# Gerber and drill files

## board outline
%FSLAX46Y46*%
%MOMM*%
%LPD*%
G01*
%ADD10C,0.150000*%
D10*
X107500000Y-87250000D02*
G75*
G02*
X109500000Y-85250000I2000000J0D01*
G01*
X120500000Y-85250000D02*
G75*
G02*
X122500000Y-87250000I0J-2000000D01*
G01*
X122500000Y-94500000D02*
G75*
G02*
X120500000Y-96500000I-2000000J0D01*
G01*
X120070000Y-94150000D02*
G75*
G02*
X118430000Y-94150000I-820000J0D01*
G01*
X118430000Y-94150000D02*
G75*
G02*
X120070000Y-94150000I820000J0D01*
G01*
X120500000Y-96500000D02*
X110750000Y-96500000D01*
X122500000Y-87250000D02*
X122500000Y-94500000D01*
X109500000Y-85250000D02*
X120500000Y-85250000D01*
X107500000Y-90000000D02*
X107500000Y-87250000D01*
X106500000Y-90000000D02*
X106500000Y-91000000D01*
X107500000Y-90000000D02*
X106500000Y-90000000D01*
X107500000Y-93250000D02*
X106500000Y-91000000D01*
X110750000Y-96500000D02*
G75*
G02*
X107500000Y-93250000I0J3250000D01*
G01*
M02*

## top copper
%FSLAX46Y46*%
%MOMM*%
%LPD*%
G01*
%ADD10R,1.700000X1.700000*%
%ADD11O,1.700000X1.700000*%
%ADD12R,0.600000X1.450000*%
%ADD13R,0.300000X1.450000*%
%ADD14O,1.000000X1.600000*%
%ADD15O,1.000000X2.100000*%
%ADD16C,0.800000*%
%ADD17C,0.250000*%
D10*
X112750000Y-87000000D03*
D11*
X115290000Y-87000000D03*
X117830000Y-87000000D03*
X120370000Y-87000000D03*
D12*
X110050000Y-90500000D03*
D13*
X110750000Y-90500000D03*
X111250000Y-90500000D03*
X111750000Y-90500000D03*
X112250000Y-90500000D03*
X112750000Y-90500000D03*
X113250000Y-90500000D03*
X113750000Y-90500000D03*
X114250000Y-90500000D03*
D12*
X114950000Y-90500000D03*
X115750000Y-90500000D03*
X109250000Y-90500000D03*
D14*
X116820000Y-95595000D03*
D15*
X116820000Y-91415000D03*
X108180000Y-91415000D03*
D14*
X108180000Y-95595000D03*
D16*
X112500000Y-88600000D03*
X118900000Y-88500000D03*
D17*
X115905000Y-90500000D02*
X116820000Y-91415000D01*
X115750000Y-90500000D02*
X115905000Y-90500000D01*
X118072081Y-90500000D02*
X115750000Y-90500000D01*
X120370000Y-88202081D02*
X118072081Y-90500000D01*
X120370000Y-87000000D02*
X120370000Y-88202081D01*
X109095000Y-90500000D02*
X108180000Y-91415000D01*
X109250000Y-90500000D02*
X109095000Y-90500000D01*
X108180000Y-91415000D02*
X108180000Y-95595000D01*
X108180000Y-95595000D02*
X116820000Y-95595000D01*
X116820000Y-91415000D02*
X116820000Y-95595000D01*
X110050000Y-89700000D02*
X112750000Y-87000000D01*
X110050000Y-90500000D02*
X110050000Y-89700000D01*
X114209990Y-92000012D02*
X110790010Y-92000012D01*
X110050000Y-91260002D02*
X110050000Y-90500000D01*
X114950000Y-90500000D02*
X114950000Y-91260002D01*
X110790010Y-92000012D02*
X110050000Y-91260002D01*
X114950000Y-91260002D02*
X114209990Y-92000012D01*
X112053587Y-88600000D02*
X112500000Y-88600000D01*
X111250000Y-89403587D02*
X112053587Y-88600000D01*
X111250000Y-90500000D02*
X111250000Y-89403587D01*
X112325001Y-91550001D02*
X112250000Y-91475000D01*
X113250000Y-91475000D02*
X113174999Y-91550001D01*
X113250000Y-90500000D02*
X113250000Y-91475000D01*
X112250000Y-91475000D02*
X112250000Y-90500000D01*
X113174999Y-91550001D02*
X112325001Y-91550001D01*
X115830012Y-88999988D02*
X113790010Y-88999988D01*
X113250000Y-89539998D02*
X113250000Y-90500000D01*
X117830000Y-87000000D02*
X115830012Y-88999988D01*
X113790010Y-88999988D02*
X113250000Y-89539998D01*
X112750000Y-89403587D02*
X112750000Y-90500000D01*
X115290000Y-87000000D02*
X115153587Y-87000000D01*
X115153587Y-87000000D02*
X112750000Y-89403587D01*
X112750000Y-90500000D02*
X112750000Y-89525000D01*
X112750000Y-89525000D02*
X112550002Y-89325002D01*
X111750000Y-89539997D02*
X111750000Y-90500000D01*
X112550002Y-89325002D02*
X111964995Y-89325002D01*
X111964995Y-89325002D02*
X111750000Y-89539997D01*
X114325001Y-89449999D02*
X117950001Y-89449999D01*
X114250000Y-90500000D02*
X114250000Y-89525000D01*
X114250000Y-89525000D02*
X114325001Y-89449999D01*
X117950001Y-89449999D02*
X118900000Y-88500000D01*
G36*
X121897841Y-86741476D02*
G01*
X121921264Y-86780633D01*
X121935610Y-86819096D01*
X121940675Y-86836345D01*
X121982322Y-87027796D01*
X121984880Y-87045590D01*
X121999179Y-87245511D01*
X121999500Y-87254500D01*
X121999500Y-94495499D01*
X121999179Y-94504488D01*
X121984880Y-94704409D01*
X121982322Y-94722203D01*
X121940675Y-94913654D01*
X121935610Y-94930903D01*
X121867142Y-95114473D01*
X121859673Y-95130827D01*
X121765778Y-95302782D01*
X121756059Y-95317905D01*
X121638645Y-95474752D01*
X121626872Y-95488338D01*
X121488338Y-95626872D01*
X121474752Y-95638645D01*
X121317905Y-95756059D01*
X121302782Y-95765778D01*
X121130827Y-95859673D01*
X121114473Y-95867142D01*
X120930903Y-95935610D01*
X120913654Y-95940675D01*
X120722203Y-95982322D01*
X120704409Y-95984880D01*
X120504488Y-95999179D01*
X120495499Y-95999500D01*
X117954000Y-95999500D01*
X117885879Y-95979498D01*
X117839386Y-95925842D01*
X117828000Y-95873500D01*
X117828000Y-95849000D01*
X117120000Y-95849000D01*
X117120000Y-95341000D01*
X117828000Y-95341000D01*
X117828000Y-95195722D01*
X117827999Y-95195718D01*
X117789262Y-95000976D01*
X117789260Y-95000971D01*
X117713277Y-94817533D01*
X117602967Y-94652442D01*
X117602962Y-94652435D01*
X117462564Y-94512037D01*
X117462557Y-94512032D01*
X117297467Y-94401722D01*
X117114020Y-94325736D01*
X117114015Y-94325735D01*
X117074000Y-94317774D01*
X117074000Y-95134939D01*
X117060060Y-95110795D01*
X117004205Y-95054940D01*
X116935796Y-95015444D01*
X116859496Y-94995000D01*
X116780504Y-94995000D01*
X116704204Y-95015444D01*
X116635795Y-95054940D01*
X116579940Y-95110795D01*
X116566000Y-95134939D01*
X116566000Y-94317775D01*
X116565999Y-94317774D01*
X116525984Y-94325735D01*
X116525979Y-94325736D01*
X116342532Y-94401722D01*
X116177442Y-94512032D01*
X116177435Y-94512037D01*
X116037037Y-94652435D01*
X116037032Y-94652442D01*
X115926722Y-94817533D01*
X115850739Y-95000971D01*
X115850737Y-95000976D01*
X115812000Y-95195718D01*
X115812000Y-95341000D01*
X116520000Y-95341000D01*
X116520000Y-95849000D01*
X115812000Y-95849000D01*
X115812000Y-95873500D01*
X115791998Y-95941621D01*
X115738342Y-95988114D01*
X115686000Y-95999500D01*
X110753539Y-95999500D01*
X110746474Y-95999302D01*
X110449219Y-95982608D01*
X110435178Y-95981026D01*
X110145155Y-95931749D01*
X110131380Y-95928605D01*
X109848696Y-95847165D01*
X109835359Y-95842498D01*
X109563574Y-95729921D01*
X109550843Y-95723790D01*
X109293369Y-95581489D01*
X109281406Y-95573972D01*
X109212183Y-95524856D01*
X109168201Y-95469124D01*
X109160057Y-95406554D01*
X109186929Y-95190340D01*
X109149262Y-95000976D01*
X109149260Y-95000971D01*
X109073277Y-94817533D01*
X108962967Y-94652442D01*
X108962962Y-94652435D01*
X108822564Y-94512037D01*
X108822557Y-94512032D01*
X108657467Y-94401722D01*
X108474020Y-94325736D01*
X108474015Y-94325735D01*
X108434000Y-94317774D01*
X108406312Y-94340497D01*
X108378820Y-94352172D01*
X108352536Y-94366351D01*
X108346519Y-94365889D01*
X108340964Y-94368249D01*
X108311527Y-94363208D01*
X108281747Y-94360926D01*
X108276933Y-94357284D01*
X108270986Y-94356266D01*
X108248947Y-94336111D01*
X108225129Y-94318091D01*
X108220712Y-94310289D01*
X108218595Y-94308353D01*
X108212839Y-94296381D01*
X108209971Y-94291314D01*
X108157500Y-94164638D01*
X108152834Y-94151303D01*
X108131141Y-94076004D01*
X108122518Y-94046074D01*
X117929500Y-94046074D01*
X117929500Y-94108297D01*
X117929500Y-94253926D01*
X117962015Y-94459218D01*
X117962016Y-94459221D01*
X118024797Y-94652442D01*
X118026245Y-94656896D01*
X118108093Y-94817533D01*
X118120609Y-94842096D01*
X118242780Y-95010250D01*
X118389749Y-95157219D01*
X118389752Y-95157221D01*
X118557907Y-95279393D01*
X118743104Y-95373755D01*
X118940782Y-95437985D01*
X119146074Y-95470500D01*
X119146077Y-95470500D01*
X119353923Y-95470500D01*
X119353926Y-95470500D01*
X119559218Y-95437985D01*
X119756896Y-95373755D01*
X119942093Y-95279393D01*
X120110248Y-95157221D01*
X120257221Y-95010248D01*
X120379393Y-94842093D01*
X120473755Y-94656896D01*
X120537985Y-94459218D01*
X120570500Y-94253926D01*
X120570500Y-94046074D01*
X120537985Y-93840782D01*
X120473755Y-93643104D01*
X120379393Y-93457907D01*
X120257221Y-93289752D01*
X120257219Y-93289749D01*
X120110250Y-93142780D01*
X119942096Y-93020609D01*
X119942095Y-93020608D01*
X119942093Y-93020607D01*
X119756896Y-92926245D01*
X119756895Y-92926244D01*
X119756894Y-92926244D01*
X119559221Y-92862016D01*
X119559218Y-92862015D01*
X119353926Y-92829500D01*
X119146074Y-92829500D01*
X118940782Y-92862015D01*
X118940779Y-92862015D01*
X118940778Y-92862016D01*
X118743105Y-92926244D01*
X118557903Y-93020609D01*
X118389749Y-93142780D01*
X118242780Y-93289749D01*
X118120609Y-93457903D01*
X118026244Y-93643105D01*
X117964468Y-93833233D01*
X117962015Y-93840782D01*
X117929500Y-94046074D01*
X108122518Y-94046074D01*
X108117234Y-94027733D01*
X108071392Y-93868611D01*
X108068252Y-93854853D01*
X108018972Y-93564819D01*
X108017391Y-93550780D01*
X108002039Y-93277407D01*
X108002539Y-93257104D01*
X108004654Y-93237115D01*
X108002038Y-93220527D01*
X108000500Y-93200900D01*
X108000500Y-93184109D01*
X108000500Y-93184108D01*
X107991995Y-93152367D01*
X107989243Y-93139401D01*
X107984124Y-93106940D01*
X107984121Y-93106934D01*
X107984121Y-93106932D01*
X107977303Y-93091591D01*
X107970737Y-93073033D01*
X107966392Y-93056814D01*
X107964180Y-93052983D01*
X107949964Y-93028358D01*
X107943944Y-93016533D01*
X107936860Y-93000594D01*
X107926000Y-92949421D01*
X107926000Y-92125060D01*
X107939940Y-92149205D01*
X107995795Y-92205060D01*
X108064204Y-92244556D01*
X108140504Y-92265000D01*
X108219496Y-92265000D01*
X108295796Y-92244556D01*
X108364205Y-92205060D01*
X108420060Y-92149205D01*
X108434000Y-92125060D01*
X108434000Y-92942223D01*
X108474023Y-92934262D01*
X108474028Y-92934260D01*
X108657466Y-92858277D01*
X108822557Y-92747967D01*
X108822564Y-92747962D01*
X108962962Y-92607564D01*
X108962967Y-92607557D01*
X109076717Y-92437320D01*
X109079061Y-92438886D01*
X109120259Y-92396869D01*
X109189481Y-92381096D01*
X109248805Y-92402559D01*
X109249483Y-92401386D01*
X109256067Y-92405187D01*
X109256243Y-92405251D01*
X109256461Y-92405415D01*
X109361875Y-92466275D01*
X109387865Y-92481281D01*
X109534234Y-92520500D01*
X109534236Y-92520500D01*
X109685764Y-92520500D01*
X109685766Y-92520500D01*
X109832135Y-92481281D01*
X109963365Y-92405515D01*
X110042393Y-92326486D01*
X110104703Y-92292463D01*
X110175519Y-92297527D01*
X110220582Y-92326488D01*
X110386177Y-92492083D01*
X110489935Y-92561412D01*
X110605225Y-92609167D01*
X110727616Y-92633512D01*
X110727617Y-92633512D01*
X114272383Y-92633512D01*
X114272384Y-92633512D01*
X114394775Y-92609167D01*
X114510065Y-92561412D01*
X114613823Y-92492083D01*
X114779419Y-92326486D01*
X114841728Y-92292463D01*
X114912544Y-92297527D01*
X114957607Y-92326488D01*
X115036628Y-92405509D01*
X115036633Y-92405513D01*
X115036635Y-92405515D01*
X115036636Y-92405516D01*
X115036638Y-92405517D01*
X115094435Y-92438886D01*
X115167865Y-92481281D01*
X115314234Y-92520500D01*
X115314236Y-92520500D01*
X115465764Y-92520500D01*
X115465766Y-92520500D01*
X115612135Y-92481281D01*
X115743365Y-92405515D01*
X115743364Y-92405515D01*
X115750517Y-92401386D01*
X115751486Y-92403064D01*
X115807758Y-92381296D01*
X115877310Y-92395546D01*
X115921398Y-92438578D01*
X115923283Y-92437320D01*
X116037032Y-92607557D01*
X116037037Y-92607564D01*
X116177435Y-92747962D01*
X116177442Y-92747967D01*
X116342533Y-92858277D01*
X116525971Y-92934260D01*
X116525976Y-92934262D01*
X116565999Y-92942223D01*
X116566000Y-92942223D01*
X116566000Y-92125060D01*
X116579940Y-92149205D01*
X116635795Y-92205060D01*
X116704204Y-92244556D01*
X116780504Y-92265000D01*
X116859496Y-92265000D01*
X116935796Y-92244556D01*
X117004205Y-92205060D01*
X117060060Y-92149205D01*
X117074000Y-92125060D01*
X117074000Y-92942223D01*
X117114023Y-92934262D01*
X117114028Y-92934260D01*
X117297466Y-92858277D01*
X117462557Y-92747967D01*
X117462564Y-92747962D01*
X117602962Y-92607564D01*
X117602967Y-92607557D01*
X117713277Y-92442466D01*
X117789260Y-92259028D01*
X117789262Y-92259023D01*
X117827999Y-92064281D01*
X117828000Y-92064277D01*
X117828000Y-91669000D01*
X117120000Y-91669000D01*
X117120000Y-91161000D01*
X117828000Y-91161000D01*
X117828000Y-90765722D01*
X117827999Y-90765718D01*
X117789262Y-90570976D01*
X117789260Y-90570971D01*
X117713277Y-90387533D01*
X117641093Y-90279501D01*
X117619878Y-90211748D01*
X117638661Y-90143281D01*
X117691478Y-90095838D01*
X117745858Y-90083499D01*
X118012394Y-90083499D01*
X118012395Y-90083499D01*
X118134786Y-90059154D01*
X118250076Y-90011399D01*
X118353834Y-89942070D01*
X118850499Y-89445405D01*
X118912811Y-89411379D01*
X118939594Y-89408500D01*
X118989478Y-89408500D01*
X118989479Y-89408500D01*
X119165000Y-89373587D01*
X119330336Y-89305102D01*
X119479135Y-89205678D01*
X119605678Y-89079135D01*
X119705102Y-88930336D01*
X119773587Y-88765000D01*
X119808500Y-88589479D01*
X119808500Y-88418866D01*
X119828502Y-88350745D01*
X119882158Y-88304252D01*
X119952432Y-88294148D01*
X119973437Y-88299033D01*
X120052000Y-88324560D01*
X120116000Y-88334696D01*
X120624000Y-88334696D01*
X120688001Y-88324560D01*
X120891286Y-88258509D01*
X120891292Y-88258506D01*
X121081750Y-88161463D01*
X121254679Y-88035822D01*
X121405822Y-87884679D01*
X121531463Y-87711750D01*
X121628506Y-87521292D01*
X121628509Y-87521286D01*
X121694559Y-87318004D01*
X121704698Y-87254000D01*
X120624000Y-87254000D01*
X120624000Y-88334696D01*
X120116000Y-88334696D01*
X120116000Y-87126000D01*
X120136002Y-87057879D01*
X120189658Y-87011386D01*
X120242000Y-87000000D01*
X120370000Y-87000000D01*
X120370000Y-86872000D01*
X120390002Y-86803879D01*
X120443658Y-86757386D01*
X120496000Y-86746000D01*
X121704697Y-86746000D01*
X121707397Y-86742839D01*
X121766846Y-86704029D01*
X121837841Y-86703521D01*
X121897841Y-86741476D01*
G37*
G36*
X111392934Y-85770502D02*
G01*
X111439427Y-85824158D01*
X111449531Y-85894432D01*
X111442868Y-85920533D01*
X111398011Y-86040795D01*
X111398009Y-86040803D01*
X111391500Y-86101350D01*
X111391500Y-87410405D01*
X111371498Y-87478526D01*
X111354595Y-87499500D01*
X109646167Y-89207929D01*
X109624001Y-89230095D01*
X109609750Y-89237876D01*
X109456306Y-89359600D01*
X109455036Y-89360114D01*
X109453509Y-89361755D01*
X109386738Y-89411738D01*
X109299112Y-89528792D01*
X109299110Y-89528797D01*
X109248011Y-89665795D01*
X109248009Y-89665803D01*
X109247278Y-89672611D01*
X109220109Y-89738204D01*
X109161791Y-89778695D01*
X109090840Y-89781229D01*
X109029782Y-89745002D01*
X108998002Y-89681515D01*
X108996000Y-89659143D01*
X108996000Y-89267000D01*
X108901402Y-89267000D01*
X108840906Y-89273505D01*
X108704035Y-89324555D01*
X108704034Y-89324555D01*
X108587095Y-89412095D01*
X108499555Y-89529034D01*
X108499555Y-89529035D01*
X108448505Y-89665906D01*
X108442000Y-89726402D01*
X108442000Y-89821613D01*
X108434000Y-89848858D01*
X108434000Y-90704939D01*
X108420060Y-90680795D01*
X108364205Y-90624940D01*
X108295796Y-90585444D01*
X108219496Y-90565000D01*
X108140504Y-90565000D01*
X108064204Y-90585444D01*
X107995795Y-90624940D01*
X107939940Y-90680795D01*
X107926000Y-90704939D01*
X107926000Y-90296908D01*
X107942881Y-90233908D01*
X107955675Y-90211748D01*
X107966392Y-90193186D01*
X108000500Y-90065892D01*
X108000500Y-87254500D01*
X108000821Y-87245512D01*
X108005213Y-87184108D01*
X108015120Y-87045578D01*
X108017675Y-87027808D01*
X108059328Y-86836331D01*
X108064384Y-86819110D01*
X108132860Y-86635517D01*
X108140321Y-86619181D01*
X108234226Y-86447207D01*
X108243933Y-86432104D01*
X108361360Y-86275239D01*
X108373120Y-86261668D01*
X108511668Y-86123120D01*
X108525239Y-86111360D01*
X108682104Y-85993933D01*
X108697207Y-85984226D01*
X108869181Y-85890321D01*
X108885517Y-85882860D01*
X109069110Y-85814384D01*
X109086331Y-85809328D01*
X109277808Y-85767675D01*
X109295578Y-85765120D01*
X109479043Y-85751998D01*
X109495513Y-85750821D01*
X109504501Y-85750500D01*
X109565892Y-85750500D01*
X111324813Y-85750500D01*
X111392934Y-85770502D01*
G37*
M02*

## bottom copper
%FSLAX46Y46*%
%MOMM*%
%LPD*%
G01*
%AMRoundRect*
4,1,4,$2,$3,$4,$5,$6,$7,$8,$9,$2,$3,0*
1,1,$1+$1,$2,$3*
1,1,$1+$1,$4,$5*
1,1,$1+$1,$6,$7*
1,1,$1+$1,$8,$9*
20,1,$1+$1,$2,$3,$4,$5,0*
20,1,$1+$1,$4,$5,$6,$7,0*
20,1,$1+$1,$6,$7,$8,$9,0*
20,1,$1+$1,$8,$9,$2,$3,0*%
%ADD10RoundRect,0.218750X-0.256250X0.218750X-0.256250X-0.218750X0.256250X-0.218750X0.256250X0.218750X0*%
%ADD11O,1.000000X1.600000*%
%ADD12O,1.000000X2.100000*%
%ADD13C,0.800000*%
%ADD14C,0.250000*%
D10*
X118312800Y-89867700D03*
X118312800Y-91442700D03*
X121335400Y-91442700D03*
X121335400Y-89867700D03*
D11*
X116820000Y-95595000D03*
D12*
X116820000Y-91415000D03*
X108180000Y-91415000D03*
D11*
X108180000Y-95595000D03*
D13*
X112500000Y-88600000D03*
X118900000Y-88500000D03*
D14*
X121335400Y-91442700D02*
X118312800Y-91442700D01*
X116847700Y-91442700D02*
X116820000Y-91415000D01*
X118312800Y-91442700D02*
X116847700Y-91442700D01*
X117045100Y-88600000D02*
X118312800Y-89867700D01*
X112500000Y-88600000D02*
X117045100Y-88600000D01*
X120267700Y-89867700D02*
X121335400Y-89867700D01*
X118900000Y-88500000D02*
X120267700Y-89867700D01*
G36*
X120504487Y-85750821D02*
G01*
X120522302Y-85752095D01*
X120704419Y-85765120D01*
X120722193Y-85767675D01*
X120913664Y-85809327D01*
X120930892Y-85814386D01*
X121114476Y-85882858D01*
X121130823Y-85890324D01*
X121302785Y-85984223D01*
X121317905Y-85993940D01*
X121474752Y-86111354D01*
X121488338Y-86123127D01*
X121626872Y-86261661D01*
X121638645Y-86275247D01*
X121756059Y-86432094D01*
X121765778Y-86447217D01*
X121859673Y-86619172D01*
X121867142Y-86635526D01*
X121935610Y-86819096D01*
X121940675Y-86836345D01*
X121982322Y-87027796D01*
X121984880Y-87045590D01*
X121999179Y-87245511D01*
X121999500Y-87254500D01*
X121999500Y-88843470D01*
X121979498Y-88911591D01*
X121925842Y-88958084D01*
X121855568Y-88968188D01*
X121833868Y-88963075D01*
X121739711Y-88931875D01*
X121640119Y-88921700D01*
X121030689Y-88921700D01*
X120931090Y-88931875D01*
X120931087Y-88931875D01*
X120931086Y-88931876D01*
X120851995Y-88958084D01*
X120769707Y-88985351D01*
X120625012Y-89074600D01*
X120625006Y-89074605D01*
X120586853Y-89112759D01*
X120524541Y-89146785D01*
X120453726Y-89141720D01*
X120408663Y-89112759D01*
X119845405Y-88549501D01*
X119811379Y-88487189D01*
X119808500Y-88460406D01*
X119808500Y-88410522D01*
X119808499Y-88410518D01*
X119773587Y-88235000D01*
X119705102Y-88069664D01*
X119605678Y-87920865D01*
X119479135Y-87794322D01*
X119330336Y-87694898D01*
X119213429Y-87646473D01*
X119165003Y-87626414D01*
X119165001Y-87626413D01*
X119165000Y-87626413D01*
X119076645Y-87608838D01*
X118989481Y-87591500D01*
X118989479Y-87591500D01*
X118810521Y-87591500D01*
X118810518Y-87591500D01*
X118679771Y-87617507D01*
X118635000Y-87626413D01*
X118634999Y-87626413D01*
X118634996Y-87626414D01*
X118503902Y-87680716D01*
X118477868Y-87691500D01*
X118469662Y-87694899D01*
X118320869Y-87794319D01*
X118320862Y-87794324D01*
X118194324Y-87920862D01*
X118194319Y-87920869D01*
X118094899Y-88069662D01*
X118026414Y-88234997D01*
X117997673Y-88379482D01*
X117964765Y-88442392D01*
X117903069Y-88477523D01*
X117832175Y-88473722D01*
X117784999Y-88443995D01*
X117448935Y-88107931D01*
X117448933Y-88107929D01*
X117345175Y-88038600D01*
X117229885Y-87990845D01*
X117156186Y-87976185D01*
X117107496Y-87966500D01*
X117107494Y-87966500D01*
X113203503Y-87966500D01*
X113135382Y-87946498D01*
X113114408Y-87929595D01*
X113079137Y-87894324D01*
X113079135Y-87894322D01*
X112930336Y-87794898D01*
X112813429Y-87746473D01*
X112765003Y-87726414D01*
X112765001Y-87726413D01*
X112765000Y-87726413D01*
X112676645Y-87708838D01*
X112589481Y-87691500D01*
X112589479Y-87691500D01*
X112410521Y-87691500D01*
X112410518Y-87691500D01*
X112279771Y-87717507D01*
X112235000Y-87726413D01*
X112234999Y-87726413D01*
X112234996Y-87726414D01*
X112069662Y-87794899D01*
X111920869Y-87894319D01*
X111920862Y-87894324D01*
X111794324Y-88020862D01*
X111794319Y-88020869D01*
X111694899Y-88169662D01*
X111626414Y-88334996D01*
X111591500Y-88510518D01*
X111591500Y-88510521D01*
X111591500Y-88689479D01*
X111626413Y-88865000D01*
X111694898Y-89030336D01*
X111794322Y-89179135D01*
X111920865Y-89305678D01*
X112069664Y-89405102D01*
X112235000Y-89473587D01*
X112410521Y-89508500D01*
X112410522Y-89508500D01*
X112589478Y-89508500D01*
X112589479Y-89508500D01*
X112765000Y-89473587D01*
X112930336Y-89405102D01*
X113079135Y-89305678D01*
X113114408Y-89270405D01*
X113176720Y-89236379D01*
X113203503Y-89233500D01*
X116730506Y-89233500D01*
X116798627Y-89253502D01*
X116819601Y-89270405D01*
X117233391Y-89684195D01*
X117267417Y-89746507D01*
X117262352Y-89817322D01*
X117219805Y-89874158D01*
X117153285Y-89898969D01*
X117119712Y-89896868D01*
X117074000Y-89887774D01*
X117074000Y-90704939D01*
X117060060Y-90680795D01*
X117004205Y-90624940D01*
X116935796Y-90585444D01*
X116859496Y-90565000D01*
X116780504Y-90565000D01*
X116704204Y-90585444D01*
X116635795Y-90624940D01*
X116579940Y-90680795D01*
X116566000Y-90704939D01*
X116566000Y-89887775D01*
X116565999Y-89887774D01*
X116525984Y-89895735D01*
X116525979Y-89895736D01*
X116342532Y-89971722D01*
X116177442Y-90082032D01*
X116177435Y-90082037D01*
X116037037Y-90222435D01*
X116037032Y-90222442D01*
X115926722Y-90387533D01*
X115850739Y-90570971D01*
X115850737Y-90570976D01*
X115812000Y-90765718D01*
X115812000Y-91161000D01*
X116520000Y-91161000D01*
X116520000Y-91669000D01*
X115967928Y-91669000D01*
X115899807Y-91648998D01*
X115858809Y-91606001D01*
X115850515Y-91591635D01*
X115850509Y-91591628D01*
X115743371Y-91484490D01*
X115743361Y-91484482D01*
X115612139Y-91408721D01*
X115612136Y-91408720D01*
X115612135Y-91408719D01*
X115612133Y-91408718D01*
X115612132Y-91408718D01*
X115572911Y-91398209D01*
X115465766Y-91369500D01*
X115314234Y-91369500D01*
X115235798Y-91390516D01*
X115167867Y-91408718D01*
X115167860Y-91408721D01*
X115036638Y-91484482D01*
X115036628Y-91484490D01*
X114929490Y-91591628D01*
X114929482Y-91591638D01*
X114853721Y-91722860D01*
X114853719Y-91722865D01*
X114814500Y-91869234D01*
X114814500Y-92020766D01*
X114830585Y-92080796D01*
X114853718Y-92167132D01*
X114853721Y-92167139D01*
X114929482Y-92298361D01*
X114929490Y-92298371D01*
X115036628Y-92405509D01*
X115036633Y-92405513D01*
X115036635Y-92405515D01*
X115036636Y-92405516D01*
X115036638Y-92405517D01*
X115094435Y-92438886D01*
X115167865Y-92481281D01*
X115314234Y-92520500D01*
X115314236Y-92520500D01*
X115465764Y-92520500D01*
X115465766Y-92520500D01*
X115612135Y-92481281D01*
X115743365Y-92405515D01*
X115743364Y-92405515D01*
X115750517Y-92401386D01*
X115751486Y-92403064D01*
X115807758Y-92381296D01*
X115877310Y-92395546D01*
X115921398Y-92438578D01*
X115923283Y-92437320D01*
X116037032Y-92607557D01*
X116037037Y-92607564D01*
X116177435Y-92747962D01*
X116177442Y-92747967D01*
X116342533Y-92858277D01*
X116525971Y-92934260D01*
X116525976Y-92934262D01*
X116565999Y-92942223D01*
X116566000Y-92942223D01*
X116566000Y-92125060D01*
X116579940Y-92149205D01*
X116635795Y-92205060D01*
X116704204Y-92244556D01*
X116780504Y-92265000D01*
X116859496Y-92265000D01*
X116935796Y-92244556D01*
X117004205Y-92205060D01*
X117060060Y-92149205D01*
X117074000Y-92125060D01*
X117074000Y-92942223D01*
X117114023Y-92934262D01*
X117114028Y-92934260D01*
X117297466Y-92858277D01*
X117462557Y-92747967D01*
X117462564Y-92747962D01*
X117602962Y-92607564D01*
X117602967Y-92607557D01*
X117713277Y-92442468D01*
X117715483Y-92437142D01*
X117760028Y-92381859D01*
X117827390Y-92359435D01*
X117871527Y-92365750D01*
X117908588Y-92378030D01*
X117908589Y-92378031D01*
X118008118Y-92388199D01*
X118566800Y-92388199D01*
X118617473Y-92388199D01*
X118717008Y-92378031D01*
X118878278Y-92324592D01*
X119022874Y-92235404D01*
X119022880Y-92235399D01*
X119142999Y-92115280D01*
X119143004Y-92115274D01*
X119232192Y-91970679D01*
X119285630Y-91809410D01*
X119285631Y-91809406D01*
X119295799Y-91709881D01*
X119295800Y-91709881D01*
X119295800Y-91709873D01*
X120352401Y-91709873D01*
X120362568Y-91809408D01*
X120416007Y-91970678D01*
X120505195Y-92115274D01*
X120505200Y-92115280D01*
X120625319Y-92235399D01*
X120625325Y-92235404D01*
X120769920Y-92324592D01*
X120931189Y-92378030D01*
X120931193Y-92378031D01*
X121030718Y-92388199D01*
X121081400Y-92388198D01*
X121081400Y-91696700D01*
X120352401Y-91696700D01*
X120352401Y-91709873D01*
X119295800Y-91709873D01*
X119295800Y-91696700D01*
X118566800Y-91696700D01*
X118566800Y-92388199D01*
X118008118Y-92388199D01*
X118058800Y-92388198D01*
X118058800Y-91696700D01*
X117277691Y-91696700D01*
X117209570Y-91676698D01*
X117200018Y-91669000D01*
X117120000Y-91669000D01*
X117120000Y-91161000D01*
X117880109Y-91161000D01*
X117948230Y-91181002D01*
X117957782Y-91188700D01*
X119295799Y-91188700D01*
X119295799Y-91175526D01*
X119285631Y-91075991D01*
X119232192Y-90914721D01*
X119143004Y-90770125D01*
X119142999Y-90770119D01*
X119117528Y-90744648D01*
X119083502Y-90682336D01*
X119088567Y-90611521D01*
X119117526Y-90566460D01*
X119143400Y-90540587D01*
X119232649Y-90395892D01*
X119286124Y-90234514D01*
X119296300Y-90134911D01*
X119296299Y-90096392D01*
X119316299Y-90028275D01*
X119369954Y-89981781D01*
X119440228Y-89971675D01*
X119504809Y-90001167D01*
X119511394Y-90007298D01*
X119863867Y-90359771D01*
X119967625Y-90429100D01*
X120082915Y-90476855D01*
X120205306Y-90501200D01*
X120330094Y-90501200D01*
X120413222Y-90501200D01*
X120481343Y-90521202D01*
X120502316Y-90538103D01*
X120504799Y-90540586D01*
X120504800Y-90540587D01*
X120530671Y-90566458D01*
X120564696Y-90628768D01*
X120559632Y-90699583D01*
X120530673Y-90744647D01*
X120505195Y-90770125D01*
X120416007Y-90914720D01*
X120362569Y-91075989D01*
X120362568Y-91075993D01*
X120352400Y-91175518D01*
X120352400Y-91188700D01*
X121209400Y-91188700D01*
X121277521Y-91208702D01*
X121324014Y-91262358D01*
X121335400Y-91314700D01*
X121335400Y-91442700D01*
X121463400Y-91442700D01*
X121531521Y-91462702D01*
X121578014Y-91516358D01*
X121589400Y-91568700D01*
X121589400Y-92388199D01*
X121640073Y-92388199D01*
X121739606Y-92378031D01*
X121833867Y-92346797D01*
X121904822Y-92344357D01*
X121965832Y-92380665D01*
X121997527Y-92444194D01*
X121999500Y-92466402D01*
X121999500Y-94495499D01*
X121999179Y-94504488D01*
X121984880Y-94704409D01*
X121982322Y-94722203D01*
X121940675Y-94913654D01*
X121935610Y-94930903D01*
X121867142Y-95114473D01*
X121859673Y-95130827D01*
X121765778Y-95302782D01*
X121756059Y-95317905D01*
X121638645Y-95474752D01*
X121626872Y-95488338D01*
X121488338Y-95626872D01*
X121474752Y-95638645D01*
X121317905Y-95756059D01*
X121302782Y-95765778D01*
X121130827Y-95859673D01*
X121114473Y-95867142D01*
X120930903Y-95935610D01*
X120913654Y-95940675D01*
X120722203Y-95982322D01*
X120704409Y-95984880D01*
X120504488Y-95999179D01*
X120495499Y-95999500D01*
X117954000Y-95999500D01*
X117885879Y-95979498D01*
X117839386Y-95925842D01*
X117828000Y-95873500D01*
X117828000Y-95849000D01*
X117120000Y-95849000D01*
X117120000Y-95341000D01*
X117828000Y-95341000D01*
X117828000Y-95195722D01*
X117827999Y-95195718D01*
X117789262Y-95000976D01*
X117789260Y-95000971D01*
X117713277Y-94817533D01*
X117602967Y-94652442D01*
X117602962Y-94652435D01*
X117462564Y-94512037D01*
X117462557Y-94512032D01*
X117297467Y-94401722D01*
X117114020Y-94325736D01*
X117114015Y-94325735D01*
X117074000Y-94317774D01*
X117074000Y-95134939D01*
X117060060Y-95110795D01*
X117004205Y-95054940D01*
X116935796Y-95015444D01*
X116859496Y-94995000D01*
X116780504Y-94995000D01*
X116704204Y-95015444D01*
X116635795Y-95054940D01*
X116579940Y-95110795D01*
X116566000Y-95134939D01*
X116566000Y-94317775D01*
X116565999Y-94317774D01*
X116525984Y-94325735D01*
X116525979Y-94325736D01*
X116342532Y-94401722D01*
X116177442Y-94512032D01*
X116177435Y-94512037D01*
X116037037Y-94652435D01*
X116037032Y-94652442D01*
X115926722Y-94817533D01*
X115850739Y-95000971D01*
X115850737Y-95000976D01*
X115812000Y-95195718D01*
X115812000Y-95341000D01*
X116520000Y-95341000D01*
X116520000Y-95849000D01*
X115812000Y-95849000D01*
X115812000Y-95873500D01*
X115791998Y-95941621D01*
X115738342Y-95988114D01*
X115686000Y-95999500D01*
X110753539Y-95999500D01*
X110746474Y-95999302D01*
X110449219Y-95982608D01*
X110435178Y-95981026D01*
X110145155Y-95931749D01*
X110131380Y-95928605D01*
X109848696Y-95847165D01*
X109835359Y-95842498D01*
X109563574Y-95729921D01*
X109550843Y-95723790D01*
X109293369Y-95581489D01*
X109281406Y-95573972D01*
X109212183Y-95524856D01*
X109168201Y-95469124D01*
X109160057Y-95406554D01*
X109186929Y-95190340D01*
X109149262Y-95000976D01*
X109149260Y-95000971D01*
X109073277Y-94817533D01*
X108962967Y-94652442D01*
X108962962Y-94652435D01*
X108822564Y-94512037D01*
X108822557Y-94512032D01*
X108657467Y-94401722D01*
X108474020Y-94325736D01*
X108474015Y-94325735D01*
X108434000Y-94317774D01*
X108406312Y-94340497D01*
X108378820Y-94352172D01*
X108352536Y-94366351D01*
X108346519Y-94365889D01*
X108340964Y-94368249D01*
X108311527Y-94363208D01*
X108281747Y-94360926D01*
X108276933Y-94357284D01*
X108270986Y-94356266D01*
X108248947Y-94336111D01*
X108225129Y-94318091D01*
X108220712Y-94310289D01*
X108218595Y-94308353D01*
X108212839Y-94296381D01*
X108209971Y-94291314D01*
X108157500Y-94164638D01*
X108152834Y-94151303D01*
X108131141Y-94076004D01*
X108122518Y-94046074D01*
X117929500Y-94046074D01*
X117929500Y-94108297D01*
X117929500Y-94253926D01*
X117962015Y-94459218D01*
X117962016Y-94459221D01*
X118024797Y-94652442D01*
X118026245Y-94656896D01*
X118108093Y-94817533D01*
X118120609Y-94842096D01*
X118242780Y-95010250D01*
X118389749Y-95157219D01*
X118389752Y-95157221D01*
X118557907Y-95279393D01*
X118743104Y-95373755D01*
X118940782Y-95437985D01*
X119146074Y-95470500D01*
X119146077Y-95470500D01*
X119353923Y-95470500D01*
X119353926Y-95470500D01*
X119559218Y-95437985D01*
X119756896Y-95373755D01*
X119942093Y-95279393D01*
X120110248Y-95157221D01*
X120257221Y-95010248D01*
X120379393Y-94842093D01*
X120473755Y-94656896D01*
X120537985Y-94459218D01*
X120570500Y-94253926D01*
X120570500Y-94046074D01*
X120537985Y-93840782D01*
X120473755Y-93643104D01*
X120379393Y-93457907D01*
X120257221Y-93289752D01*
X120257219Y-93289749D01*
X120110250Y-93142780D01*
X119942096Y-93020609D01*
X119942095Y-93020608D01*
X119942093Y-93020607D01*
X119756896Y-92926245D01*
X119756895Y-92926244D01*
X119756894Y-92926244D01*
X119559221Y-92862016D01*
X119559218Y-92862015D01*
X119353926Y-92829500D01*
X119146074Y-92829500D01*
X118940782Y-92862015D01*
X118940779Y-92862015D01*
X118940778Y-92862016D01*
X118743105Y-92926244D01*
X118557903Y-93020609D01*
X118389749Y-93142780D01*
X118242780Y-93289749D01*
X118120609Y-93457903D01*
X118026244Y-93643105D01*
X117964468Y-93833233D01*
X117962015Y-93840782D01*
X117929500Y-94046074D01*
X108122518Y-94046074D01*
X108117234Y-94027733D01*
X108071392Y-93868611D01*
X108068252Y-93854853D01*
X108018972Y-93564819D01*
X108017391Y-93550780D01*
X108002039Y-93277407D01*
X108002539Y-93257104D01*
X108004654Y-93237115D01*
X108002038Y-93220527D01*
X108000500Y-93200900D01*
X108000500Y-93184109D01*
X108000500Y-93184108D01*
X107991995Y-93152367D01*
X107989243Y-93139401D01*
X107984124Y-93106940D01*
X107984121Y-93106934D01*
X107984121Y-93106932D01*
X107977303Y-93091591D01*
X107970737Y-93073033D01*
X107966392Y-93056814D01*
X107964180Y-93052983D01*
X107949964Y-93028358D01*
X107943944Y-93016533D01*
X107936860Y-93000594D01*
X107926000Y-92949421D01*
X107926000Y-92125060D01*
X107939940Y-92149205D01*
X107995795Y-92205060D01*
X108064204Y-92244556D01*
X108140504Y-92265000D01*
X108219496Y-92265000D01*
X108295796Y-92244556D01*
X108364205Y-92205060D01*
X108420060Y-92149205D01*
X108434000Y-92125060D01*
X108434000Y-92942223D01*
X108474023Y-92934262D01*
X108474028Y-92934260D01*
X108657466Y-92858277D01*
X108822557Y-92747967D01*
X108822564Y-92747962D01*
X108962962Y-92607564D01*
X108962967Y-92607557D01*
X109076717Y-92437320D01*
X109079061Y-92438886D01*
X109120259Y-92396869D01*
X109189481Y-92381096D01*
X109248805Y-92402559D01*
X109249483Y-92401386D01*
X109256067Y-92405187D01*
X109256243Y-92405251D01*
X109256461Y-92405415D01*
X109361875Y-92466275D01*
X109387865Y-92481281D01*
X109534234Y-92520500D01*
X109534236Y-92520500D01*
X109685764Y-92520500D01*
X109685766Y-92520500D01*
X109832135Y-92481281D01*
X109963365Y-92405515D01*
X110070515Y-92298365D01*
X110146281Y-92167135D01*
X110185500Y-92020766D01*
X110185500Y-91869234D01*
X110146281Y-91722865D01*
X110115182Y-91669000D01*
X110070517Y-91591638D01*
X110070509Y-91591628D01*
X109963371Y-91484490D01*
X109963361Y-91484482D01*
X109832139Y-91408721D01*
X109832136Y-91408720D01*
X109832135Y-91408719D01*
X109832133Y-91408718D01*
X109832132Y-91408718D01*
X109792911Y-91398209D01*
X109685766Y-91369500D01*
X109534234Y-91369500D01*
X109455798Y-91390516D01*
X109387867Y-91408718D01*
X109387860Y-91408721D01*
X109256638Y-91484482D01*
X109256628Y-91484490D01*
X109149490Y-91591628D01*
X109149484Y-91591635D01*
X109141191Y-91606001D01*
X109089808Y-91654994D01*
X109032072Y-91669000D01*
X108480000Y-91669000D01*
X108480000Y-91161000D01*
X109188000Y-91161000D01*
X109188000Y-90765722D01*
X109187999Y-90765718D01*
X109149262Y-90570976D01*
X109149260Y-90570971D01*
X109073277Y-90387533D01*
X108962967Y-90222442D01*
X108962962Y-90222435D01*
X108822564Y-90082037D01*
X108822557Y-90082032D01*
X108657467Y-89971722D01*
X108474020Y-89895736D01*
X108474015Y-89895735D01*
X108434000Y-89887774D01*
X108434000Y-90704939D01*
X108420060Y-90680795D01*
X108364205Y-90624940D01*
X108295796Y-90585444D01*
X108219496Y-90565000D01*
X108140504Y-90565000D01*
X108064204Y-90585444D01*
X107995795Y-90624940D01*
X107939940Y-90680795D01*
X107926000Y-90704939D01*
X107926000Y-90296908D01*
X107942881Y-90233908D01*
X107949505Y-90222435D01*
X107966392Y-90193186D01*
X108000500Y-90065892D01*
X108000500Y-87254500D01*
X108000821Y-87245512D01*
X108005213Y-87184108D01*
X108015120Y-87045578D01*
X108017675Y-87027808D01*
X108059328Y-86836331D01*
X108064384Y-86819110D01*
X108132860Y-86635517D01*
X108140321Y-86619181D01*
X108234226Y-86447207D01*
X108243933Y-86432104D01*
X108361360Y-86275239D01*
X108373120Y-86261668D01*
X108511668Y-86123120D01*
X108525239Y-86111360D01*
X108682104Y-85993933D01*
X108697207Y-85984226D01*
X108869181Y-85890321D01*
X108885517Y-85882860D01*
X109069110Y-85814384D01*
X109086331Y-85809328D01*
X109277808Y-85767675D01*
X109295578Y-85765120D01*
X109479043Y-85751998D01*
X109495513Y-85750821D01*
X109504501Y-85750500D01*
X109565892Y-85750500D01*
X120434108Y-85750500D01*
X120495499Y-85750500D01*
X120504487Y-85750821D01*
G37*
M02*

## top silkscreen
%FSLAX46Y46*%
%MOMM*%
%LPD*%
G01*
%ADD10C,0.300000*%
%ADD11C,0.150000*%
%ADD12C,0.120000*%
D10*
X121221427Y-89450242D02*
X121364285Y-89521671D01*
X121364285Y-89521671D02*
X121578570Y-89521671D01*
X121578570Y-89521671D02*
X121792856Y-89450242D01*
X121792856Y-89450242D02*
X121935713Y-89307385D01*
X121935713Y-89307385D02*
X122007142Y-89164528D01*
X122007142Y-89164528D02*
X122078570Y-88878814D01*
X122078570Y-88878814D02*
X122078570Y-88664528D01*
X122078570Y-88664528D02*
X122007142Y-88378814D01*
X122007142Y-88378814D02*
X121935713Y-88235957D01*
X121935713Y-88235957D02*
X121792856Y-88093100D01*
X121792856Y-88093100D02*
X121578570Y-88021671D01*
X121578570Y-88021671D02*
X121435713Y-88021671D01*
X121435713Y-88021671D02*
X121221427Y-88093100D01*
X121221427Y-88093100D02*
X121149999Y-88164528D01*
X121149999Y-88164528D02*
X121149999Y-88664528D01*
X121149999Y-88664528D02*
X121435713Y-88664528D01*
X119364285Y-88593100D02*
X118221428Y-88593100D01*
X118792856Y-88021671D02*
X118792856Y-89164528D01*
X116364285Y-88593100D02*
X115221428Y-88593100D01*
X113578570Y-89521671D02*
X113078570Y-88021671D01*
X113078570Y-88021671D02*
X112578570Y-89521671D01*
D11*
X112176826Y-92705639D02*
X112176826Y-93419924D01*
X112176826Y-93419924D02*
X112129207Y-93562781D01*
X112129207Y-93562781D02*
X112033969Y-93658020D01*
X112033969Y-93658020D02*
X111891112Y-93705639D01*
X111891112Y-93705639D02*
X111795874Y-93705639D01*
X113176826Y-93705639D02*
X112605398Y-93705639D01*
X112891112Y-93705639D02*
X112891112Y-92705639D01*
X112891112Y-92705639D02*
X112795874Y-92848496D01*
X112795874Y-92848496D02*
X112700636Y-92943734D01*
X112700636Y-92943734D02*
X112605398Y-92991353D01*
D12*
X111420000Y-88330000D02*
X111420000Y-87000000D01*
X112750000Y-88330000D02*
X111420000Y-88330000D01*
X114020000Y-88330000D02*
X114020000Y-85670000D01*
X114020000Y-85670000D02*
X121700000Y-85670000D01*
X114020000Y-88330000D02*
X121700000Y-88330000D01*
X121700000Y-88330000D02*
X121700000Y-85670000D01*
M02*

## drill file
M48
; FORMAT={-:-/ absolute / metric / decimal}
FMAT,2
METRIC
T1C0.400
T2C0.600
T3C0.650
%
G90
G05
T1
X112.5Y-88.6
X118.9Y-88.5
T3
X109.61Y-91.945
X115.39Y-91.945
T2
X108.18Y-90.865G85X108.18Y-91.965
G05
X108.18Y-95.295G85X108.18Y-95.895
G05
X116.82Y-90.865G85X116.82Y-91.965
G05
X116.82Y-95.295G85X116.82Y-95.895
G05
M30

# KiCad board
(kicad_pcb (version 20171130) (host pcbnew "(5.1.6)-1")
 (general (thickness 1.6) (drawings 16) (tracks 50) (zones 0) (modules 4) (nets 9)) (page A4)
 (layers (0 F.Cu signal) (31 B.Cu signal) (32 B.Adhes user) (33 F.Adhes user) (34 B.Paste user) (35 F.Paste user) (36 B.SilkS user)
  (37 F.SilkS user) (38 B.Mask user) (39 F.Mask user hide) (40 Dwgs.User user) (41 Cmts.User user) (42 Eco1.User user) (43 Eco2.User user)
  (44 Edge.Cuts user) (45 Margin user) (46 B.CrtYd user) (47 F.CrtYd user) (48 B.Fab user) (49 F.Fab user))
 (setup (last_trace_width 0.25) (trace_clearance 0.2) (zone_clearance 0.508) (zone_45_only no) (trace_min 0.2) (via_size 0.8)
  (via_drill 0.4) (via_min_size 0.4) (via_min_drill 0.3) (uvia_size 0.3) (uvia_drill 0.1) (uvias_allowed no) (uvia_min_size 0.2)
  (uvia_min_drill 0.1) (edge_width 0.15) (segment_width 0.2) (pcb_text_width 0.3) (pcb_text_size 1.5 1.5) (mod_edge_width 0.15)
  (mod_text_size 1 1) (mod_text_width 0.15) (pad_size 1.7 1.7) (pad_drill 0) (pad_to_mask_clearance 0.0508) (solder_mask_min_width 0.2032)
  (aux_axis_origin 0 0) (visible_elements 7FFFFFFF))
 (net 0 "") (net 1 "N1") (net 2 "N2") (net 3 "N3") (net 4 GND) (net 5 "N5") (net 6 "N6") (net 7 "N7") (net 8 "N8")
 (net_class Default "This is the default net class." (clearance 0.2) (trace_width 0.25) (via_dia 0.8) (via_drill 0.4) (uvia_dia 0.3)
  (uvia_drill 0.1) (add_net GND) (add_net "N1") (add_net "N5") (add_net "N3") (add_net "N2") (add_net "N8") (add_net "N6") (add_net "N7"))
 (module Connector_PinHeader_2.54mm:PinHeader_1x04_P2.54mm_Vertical (layer F.Cu) (at 112.75 87 90)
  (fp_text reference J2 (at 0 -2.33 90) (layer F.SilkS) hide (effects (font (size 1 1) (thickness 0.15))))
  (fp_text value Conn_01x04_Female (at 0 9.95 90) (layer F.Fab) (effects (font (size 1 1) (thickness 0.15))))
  (fp_line (start -1.33 -1.33) (end 0 -1.33) (layer F.SilkS) (width 0.12))
  (fp_line (start -1.33 0) (end -1.33 -1.33) (layer F.SilkS) (width 0.12))
  (fp_line (start -1.33 1.27) (end 1.33 1.27) (layer F.SilkS) (width 0.12))
  (fp_line (start 1.33 1.27) (end 1.33 8.95) (layer F.SilkS) (width 0.12))
  (fp_line (start -1.33 1.27) (end -1.33 8.95) (layer F.SilkS) (width 0.12))
  (fp_line (start -1.33 8.95) (end 1.33 8.95) (layer F.SilkS) (width 0.12))
  (pad 1 smd rect (at 0 0 90) (size 1.7 1.7) (layers F.Cu F.Paste F.Mask) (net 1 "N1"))
  (pad 2 smd oval (at 0 2.54 90) (size 1.7 1.7) (layers F.Cu F.Paste F.Mask) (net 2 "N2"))
  (pad 3 smd oval (at 0 5.08 90) (size 1.7 1.7) (layers F.Cu F.Paste F.Mask) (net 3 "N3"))
  (pad 4 smd oval (at 0 7.62 90) (size 1.7 1.7) (layers F.Cu F.Paste F.Mask) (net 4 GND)))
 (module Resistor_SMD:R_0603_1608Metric (layer B.Cu) (at 118.3128 90.6552 270)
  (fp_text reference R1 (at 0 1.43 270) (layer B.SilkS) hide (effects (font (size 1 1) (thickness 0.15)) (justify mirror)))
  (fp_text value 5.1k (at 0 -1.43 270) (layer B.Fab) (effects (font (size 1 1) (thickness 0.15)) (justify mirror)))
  (pad 1 smd roundrect (at -0.7875 0 270) (size 0.875 0.95) (layers B.Cu B.Paste B.Mask) (roundrect_rratio 0.25) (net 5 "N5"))
  (pad 2 smd roundrect (at 0.7875 0 270) (size 0.875 0.95) (layers B.Cu B.Paste B.Mask) (roundrect_rratio 0.25) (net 4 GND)))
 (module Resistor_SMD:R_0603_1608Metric (layer B.Cu) (at 121.3354 90.6552 270)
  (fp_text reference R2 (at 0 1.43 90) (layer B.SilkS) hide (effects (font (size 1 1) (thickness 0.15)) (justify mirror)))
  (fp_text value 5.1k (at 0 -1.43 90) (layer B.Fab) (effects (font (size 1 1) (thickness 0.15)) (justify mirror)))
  (pad 2 smd roundrect (at 0.7875 0 270) (size 0.875 0.95) (layers B.Cu B.Paste B.Mask) (roundrect_rratio 0.25) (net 4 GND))
  (pad 1 smd roundrect (at -0.7875 0 270) (size 0.875 0.95) (layers B.Cu B.Paste B.Mask) (roundrect_rratio 0.25) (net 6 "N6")))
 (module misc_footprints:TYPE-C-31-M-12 (layer F.Cu) (at 112.5 90.5)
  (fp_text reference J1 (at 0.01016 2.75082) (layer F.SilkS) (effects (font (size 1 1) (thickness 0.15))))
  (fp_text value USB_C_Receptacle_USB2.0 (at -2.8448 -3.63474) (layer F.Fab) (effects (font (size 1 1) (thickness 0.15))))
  (pad A4|B9 smd rect (at -2.45 0) (size 0.6 1.45) (layers F.Cu F.Paste F.Mask) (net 1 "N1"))
  (pad B8 smd rect (at -1.75 0) (size 0.3 1.45) (layers F.Cu F.Paste F.Mask) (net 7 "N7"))
  (pad A5 smd rect (at -1.25 0) (size 0.3 1.45) (layers F.Cu F.Paste F.Mask) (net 5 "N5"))
  (pad B7 smd rect (at -0.75 0) (size 0.3 1.45) (layers F.Cu F.Paste F.Mask) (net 2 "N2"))
  (pad A6 smd rect (at -0.25 0) (size 0.3 1.45) (layers F.Cu F.Paste F.Mask) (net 3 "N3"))
  (pad A7 smd rect (at 0.25 0) (size 0.3 1.45) (layers F.Cu F.Paste F.Mask) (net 2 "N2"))
  (pad B6 smd rect (at 0.75 0) (size 0.3 1.45) (layers F.Cu F.Paste F.Mask) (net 3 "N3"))
  (pad A8 smd rect (at 1.25 0) (size 0.3 1.45) (layers F.Cu F.Paste F.Mask) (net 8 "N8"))
  (pad B5 smd rect (at 1.75 0) (size 0.3 1.45) (layers F.Cu F.Paste F.Mask) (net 6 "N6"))
  (pad B4|A9 smd rect (at 2.45 0) (size 0.6 1.45) (layers F.Cu F.Paste F.Mask) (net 1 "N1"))
  (pad B1|A12 smd rect (at 3.25 0) (size 0.6 1.45) (layers F.Cu F.Paste F.Mask) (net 4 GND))
  (pad A1|B12 smd rect (at -3.25 0) (size 0.6 1.45) (layers F.Cu F.Paste F.Mask) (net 4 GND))
  (pad GND thru_hole oval (at 4.32 5.095) (size 1 1.6) (drill oval 0.6 1.2) (layers *.Cu *.Mask) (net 4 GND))
  (pad GND thru_hole oval (at 4.32 0.915) (size 1 2.1) (drill oval 0.6 1.7) (layers *.Cu *.Mask) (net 4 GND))
  (pad GND thru_hole oval (at -4.32 0.915) (size 1 2.1) (drill oval 0.6 1.7) (layers *.Cu *.Mask) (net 4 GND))
  (pad GND thru_hole oval (at -4.32 5.095) (size 1 1.6) (drill oval 0.6 1.2) (layers *.Cu *.Mask) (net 4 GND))
  (pad "" np_thru_hole circle (at 2.89 1.445) (size 0.65 0.65) (drill 0.65) (layers *.Cu *.Mask))
  (pad "" np_thru_hole circle (at -2.89 1.445) (size 0.65 0.65) (drill 0.65) (layers *.Cu *.Mask)))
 (gr_arc (start 109.5 87.25) (end 109.5 85.25) (angle -90) (layer Edge.Cuts) (width 0.15))
 (gr_arc (start 120.5 87.25) (end 122.5 87.25) (angle -90) (layer Edge.Cuts) (width 0.15))
 (gr_arc (start 120.5 94.5) (end 120.5 96.5) (angle -90) (layer Edge.Cuts) (width 0.15))
 (gr_circle (center 119.25 94.15) (end 120.07 94.15) (layer Edge.Cuts) (width 0.15))
 (gr_line (start 120.5 96.5) (end 110.75 96.5) (layer Edge.Cuts) (width 0.15))
 (gr_line (start 122.5 87.25) (end 122.5 94.5) (layer Edge.Cuts) (width 0.15))
 (gr_line (start 109.5 85.25) (end 120.5 85.25) (layer Edge.Cuts) (width 0.15))
 (gr_line (start 107.5 90) (end 107.5 87.25) (layer Edge.Cuts) (width 0.15))
 (gr_line (start 106.5 90) (end 106.5 91) (layer Edge.Cuts) (width 0.15))
 (gr_line (start 107.5 90) (end 106.5 90) (layer Edge.Cuts) (width 0.15))
 (gr_line (start 107.5 93.25) (end 106.5 91) (layer Edge.Cuts) (width 0.15))
 (gr_arc (start 110.75 93.25) (end 107.5 93.25) (angle -90) (layer Edge.Cuts) (width 0.15))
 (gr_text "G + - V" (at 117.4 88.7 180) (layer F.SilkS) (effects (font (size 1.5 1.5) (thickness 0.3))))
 (segment (start 121.3354 91.4427) (end 118.3128 91.4427) (width 0.25) (layer B.Cu) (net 4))
 (segment (start 116.8477 91.4427) (end 116.82 91.415) (width 0.25) (layer B.Cu) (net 4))
 (segment (start 118.3128 91.4427) (end 116.8477 91.4427) (width 0.25) (layer B.Cu) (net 4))
 (segment (start 115.905 90.5) (end 116.82 91.415) (width 0.25) (layer F.Cu) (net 4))
 (segment (start 115.75 90.5) (end 115.905 90.5) (width 0.25) (layer F.Cu) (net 4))
 (segment (start 118.072081 90.5) (end 115.75 90.5) (width 0.25) (layer F.Cu) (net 4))
 (segment (start 120.37 88.202081) (end 118.072081 90.5) (width 0.25) (layer F.Cu) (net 4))
 (segment (start 120.37 87) (end 120.37 88.202081) (width 0.25) (layer F.Cu) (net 4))
 (segment (start 109.095 90.5) (end 108.18 91.415) (width 0.25) (layer F.Cu) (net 4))
 (segment (start 109.25 90.5) (end 109.095 90.5) (width 0.25) (layer F.Cu) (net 4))
 (segment (start 108.18 91.415) (end 108.18 95.595) (width 0.25) (layer F.Cu) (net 4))
 (segment (start 108.18 95.595) (end 116.82 95.595) (width 0.25) (layer F.Cu) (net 4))
 (segment (start 116.82 91.415) (end 116.82 95.595) (width 0.25) (layer F.Cu) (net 4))
 (segment (start 110.05 89.7) (end 112.75 87) (width 0.25) (layer F.Cu) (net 1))
 (segment (start 110.05 90.5) (end 110.05 89.7) (width 0.25) (layer F.Cu) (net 1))
 (segment (start 114.20999 92.000012) (end 110.79001 92.000012) (width 0.25) (layer F.Cu) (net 1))
 (segment (start 110.05 91.260002) (end 110.05 90.5) (width 0.25) (layer F.Cu) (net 1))
 (segment (start 114.95 90.5) (end 114.95 91.260002) (width 0.25) (layer F.Cu) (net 1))
 (segment (start 110.79001 92.000012) (end 110.05 91.260002) (width 0.25) (layer F.Cu) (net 1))
 (segment (start 114.95 91.260002) (end 114.20999 92.000012) (width 0.25) (layer F.Cu) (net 1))
 (via (at 112.5 88.6) (size 0.8) (drill 0.4) (layers F.Cu B.Cu) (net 5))
 (segment (start 112.053587 88.6) (end 112.5 88.6) (width 0.25) (layer F.Cu) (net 5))
 (segment (start 111.25 89.403587) (end 112.053587 88.6) (width 0.25) (layer F.Cu) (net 5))
 (segment (start 111.25 90.5) (end 111.25 89.403587) (width 0.25) (layer F.Cu) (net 5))
 (segment (start 117.0451 88.6) (end 118.3128 89.8677) (width 0.25) (layer B.Cu) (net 5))
 (segment (start 112.5 88.6) (end 117.0451 88.6) (width 0.25) (layer B.Cu) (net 5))
 (segment (start 112.325001 91.550001) (end 112.25 91.475) (width 0.25) (layer F.Cu) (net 3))
 (segment (start 113.25 91.475) (end 113.174999 91.550001) (width 0.25) (layer F.Cu) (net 3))
 (segment (start 113.25 90.5) (end 113.25 91.475) (width 0.25) (layer F.Cu) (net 3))
 (segment (start 112.25 91.475) (end 112.25 90.5) (width 0.25) (layer F.Cu) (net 3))
 (segment (start 113.174999 91.550001) (end 112.325001 91.550001) (width 0.25) (layer F.Cu) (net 3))
 (segment (start 115.830012 88.999988) (end 113.79001 88.999988) (width 0.25) (layer F.Cu) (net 3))
 (segment (start 113.25 89.539998) (end 113.25 90.5) (width 0.25) (layer F.Cu) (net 3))
 (segment (start 117.83 87) (end 115.830012 88.999988) (width 0.25) (layer F.Cu) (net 3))
 (segment (start 113.79001 88.999988) (end 113.25 89.539998) (width 0.25) (layer F.Cu) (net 3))
 (segment (start 112.75 89.403587) (end 112.75 90.5) (width 0.25) (layer F.Cu) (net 2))
 (segment (start 115.29 87) (end 115.153587 87) (width 0.25) (layer F.Cu) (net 2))
 (segment (start 115.153587 87) (end 112.75 89.403587) (width 0.25) (layer F.Cu) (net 2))
 (segment (start 112.75 90.5) (end 112.75 89.525) (width 0.25) (layer F.Cu) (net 2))
 (segment (start 112.75 89.525) (end 112.550002 89.325002) (width 0.25) (layer F.Cu) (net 2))
 (segment (start 111.75 89.539997) (end 111.75 90.5) (width 0.25) (layer F.Cu) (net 2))
 (segment (start 112.550002 89.325002) (end 111.964995 89.325002) (width 0.25) (layer F.Cu) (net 2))
 (segment (start 111.964995 89.325002) (end 111.75 89.539997) (width 0.25) (layer F.Cu) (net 2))
 (via (at 118.9 88.5) (size 0.8) (drill 0.4) (layers F.Cu B.Cu) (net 6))
 (segment (start 114.325001 89.449999) (end 117.950001 89.449999) (width 0.25) (layer F.Cu) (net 6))
 (segment (start 114.25 90.5) (end 114.25 89.525) (width 0.25) (layer F.Cu) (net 6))
 (segment (start 114.25 89.525) (end 114.325001 89.449999) (width 0.25) (layer F.Cu) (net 6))
 (segment (start 117.950001 89.449999) (end 118.9 88.5) (width 0.25) (layer F.Cu) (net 6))
 (segment (start 120.2677 89.8677) (end 121.3354 89.8677) (width 0.25) (layer B.Cu) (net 6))
 (segment (start 118.9 88.5) (end 120.2677 89.8677) (width 0.25) (layer B.Cu) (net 6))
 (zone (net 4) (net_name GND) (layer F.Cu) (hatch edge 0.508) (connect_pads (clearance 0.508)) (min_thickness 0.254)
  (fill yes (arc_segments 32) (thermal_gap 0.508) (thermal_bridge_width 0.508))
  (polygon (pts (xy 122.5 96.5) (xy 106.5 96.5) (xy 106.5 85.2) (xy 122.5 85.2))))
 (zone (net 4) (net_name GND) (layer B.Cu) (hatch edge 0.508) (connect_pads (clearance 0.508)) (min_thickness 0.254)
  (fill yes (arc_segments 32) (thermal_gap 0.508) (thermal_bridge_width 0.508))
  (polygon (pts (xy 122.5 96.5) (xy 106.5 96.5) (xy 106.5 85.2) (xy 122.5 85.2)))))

